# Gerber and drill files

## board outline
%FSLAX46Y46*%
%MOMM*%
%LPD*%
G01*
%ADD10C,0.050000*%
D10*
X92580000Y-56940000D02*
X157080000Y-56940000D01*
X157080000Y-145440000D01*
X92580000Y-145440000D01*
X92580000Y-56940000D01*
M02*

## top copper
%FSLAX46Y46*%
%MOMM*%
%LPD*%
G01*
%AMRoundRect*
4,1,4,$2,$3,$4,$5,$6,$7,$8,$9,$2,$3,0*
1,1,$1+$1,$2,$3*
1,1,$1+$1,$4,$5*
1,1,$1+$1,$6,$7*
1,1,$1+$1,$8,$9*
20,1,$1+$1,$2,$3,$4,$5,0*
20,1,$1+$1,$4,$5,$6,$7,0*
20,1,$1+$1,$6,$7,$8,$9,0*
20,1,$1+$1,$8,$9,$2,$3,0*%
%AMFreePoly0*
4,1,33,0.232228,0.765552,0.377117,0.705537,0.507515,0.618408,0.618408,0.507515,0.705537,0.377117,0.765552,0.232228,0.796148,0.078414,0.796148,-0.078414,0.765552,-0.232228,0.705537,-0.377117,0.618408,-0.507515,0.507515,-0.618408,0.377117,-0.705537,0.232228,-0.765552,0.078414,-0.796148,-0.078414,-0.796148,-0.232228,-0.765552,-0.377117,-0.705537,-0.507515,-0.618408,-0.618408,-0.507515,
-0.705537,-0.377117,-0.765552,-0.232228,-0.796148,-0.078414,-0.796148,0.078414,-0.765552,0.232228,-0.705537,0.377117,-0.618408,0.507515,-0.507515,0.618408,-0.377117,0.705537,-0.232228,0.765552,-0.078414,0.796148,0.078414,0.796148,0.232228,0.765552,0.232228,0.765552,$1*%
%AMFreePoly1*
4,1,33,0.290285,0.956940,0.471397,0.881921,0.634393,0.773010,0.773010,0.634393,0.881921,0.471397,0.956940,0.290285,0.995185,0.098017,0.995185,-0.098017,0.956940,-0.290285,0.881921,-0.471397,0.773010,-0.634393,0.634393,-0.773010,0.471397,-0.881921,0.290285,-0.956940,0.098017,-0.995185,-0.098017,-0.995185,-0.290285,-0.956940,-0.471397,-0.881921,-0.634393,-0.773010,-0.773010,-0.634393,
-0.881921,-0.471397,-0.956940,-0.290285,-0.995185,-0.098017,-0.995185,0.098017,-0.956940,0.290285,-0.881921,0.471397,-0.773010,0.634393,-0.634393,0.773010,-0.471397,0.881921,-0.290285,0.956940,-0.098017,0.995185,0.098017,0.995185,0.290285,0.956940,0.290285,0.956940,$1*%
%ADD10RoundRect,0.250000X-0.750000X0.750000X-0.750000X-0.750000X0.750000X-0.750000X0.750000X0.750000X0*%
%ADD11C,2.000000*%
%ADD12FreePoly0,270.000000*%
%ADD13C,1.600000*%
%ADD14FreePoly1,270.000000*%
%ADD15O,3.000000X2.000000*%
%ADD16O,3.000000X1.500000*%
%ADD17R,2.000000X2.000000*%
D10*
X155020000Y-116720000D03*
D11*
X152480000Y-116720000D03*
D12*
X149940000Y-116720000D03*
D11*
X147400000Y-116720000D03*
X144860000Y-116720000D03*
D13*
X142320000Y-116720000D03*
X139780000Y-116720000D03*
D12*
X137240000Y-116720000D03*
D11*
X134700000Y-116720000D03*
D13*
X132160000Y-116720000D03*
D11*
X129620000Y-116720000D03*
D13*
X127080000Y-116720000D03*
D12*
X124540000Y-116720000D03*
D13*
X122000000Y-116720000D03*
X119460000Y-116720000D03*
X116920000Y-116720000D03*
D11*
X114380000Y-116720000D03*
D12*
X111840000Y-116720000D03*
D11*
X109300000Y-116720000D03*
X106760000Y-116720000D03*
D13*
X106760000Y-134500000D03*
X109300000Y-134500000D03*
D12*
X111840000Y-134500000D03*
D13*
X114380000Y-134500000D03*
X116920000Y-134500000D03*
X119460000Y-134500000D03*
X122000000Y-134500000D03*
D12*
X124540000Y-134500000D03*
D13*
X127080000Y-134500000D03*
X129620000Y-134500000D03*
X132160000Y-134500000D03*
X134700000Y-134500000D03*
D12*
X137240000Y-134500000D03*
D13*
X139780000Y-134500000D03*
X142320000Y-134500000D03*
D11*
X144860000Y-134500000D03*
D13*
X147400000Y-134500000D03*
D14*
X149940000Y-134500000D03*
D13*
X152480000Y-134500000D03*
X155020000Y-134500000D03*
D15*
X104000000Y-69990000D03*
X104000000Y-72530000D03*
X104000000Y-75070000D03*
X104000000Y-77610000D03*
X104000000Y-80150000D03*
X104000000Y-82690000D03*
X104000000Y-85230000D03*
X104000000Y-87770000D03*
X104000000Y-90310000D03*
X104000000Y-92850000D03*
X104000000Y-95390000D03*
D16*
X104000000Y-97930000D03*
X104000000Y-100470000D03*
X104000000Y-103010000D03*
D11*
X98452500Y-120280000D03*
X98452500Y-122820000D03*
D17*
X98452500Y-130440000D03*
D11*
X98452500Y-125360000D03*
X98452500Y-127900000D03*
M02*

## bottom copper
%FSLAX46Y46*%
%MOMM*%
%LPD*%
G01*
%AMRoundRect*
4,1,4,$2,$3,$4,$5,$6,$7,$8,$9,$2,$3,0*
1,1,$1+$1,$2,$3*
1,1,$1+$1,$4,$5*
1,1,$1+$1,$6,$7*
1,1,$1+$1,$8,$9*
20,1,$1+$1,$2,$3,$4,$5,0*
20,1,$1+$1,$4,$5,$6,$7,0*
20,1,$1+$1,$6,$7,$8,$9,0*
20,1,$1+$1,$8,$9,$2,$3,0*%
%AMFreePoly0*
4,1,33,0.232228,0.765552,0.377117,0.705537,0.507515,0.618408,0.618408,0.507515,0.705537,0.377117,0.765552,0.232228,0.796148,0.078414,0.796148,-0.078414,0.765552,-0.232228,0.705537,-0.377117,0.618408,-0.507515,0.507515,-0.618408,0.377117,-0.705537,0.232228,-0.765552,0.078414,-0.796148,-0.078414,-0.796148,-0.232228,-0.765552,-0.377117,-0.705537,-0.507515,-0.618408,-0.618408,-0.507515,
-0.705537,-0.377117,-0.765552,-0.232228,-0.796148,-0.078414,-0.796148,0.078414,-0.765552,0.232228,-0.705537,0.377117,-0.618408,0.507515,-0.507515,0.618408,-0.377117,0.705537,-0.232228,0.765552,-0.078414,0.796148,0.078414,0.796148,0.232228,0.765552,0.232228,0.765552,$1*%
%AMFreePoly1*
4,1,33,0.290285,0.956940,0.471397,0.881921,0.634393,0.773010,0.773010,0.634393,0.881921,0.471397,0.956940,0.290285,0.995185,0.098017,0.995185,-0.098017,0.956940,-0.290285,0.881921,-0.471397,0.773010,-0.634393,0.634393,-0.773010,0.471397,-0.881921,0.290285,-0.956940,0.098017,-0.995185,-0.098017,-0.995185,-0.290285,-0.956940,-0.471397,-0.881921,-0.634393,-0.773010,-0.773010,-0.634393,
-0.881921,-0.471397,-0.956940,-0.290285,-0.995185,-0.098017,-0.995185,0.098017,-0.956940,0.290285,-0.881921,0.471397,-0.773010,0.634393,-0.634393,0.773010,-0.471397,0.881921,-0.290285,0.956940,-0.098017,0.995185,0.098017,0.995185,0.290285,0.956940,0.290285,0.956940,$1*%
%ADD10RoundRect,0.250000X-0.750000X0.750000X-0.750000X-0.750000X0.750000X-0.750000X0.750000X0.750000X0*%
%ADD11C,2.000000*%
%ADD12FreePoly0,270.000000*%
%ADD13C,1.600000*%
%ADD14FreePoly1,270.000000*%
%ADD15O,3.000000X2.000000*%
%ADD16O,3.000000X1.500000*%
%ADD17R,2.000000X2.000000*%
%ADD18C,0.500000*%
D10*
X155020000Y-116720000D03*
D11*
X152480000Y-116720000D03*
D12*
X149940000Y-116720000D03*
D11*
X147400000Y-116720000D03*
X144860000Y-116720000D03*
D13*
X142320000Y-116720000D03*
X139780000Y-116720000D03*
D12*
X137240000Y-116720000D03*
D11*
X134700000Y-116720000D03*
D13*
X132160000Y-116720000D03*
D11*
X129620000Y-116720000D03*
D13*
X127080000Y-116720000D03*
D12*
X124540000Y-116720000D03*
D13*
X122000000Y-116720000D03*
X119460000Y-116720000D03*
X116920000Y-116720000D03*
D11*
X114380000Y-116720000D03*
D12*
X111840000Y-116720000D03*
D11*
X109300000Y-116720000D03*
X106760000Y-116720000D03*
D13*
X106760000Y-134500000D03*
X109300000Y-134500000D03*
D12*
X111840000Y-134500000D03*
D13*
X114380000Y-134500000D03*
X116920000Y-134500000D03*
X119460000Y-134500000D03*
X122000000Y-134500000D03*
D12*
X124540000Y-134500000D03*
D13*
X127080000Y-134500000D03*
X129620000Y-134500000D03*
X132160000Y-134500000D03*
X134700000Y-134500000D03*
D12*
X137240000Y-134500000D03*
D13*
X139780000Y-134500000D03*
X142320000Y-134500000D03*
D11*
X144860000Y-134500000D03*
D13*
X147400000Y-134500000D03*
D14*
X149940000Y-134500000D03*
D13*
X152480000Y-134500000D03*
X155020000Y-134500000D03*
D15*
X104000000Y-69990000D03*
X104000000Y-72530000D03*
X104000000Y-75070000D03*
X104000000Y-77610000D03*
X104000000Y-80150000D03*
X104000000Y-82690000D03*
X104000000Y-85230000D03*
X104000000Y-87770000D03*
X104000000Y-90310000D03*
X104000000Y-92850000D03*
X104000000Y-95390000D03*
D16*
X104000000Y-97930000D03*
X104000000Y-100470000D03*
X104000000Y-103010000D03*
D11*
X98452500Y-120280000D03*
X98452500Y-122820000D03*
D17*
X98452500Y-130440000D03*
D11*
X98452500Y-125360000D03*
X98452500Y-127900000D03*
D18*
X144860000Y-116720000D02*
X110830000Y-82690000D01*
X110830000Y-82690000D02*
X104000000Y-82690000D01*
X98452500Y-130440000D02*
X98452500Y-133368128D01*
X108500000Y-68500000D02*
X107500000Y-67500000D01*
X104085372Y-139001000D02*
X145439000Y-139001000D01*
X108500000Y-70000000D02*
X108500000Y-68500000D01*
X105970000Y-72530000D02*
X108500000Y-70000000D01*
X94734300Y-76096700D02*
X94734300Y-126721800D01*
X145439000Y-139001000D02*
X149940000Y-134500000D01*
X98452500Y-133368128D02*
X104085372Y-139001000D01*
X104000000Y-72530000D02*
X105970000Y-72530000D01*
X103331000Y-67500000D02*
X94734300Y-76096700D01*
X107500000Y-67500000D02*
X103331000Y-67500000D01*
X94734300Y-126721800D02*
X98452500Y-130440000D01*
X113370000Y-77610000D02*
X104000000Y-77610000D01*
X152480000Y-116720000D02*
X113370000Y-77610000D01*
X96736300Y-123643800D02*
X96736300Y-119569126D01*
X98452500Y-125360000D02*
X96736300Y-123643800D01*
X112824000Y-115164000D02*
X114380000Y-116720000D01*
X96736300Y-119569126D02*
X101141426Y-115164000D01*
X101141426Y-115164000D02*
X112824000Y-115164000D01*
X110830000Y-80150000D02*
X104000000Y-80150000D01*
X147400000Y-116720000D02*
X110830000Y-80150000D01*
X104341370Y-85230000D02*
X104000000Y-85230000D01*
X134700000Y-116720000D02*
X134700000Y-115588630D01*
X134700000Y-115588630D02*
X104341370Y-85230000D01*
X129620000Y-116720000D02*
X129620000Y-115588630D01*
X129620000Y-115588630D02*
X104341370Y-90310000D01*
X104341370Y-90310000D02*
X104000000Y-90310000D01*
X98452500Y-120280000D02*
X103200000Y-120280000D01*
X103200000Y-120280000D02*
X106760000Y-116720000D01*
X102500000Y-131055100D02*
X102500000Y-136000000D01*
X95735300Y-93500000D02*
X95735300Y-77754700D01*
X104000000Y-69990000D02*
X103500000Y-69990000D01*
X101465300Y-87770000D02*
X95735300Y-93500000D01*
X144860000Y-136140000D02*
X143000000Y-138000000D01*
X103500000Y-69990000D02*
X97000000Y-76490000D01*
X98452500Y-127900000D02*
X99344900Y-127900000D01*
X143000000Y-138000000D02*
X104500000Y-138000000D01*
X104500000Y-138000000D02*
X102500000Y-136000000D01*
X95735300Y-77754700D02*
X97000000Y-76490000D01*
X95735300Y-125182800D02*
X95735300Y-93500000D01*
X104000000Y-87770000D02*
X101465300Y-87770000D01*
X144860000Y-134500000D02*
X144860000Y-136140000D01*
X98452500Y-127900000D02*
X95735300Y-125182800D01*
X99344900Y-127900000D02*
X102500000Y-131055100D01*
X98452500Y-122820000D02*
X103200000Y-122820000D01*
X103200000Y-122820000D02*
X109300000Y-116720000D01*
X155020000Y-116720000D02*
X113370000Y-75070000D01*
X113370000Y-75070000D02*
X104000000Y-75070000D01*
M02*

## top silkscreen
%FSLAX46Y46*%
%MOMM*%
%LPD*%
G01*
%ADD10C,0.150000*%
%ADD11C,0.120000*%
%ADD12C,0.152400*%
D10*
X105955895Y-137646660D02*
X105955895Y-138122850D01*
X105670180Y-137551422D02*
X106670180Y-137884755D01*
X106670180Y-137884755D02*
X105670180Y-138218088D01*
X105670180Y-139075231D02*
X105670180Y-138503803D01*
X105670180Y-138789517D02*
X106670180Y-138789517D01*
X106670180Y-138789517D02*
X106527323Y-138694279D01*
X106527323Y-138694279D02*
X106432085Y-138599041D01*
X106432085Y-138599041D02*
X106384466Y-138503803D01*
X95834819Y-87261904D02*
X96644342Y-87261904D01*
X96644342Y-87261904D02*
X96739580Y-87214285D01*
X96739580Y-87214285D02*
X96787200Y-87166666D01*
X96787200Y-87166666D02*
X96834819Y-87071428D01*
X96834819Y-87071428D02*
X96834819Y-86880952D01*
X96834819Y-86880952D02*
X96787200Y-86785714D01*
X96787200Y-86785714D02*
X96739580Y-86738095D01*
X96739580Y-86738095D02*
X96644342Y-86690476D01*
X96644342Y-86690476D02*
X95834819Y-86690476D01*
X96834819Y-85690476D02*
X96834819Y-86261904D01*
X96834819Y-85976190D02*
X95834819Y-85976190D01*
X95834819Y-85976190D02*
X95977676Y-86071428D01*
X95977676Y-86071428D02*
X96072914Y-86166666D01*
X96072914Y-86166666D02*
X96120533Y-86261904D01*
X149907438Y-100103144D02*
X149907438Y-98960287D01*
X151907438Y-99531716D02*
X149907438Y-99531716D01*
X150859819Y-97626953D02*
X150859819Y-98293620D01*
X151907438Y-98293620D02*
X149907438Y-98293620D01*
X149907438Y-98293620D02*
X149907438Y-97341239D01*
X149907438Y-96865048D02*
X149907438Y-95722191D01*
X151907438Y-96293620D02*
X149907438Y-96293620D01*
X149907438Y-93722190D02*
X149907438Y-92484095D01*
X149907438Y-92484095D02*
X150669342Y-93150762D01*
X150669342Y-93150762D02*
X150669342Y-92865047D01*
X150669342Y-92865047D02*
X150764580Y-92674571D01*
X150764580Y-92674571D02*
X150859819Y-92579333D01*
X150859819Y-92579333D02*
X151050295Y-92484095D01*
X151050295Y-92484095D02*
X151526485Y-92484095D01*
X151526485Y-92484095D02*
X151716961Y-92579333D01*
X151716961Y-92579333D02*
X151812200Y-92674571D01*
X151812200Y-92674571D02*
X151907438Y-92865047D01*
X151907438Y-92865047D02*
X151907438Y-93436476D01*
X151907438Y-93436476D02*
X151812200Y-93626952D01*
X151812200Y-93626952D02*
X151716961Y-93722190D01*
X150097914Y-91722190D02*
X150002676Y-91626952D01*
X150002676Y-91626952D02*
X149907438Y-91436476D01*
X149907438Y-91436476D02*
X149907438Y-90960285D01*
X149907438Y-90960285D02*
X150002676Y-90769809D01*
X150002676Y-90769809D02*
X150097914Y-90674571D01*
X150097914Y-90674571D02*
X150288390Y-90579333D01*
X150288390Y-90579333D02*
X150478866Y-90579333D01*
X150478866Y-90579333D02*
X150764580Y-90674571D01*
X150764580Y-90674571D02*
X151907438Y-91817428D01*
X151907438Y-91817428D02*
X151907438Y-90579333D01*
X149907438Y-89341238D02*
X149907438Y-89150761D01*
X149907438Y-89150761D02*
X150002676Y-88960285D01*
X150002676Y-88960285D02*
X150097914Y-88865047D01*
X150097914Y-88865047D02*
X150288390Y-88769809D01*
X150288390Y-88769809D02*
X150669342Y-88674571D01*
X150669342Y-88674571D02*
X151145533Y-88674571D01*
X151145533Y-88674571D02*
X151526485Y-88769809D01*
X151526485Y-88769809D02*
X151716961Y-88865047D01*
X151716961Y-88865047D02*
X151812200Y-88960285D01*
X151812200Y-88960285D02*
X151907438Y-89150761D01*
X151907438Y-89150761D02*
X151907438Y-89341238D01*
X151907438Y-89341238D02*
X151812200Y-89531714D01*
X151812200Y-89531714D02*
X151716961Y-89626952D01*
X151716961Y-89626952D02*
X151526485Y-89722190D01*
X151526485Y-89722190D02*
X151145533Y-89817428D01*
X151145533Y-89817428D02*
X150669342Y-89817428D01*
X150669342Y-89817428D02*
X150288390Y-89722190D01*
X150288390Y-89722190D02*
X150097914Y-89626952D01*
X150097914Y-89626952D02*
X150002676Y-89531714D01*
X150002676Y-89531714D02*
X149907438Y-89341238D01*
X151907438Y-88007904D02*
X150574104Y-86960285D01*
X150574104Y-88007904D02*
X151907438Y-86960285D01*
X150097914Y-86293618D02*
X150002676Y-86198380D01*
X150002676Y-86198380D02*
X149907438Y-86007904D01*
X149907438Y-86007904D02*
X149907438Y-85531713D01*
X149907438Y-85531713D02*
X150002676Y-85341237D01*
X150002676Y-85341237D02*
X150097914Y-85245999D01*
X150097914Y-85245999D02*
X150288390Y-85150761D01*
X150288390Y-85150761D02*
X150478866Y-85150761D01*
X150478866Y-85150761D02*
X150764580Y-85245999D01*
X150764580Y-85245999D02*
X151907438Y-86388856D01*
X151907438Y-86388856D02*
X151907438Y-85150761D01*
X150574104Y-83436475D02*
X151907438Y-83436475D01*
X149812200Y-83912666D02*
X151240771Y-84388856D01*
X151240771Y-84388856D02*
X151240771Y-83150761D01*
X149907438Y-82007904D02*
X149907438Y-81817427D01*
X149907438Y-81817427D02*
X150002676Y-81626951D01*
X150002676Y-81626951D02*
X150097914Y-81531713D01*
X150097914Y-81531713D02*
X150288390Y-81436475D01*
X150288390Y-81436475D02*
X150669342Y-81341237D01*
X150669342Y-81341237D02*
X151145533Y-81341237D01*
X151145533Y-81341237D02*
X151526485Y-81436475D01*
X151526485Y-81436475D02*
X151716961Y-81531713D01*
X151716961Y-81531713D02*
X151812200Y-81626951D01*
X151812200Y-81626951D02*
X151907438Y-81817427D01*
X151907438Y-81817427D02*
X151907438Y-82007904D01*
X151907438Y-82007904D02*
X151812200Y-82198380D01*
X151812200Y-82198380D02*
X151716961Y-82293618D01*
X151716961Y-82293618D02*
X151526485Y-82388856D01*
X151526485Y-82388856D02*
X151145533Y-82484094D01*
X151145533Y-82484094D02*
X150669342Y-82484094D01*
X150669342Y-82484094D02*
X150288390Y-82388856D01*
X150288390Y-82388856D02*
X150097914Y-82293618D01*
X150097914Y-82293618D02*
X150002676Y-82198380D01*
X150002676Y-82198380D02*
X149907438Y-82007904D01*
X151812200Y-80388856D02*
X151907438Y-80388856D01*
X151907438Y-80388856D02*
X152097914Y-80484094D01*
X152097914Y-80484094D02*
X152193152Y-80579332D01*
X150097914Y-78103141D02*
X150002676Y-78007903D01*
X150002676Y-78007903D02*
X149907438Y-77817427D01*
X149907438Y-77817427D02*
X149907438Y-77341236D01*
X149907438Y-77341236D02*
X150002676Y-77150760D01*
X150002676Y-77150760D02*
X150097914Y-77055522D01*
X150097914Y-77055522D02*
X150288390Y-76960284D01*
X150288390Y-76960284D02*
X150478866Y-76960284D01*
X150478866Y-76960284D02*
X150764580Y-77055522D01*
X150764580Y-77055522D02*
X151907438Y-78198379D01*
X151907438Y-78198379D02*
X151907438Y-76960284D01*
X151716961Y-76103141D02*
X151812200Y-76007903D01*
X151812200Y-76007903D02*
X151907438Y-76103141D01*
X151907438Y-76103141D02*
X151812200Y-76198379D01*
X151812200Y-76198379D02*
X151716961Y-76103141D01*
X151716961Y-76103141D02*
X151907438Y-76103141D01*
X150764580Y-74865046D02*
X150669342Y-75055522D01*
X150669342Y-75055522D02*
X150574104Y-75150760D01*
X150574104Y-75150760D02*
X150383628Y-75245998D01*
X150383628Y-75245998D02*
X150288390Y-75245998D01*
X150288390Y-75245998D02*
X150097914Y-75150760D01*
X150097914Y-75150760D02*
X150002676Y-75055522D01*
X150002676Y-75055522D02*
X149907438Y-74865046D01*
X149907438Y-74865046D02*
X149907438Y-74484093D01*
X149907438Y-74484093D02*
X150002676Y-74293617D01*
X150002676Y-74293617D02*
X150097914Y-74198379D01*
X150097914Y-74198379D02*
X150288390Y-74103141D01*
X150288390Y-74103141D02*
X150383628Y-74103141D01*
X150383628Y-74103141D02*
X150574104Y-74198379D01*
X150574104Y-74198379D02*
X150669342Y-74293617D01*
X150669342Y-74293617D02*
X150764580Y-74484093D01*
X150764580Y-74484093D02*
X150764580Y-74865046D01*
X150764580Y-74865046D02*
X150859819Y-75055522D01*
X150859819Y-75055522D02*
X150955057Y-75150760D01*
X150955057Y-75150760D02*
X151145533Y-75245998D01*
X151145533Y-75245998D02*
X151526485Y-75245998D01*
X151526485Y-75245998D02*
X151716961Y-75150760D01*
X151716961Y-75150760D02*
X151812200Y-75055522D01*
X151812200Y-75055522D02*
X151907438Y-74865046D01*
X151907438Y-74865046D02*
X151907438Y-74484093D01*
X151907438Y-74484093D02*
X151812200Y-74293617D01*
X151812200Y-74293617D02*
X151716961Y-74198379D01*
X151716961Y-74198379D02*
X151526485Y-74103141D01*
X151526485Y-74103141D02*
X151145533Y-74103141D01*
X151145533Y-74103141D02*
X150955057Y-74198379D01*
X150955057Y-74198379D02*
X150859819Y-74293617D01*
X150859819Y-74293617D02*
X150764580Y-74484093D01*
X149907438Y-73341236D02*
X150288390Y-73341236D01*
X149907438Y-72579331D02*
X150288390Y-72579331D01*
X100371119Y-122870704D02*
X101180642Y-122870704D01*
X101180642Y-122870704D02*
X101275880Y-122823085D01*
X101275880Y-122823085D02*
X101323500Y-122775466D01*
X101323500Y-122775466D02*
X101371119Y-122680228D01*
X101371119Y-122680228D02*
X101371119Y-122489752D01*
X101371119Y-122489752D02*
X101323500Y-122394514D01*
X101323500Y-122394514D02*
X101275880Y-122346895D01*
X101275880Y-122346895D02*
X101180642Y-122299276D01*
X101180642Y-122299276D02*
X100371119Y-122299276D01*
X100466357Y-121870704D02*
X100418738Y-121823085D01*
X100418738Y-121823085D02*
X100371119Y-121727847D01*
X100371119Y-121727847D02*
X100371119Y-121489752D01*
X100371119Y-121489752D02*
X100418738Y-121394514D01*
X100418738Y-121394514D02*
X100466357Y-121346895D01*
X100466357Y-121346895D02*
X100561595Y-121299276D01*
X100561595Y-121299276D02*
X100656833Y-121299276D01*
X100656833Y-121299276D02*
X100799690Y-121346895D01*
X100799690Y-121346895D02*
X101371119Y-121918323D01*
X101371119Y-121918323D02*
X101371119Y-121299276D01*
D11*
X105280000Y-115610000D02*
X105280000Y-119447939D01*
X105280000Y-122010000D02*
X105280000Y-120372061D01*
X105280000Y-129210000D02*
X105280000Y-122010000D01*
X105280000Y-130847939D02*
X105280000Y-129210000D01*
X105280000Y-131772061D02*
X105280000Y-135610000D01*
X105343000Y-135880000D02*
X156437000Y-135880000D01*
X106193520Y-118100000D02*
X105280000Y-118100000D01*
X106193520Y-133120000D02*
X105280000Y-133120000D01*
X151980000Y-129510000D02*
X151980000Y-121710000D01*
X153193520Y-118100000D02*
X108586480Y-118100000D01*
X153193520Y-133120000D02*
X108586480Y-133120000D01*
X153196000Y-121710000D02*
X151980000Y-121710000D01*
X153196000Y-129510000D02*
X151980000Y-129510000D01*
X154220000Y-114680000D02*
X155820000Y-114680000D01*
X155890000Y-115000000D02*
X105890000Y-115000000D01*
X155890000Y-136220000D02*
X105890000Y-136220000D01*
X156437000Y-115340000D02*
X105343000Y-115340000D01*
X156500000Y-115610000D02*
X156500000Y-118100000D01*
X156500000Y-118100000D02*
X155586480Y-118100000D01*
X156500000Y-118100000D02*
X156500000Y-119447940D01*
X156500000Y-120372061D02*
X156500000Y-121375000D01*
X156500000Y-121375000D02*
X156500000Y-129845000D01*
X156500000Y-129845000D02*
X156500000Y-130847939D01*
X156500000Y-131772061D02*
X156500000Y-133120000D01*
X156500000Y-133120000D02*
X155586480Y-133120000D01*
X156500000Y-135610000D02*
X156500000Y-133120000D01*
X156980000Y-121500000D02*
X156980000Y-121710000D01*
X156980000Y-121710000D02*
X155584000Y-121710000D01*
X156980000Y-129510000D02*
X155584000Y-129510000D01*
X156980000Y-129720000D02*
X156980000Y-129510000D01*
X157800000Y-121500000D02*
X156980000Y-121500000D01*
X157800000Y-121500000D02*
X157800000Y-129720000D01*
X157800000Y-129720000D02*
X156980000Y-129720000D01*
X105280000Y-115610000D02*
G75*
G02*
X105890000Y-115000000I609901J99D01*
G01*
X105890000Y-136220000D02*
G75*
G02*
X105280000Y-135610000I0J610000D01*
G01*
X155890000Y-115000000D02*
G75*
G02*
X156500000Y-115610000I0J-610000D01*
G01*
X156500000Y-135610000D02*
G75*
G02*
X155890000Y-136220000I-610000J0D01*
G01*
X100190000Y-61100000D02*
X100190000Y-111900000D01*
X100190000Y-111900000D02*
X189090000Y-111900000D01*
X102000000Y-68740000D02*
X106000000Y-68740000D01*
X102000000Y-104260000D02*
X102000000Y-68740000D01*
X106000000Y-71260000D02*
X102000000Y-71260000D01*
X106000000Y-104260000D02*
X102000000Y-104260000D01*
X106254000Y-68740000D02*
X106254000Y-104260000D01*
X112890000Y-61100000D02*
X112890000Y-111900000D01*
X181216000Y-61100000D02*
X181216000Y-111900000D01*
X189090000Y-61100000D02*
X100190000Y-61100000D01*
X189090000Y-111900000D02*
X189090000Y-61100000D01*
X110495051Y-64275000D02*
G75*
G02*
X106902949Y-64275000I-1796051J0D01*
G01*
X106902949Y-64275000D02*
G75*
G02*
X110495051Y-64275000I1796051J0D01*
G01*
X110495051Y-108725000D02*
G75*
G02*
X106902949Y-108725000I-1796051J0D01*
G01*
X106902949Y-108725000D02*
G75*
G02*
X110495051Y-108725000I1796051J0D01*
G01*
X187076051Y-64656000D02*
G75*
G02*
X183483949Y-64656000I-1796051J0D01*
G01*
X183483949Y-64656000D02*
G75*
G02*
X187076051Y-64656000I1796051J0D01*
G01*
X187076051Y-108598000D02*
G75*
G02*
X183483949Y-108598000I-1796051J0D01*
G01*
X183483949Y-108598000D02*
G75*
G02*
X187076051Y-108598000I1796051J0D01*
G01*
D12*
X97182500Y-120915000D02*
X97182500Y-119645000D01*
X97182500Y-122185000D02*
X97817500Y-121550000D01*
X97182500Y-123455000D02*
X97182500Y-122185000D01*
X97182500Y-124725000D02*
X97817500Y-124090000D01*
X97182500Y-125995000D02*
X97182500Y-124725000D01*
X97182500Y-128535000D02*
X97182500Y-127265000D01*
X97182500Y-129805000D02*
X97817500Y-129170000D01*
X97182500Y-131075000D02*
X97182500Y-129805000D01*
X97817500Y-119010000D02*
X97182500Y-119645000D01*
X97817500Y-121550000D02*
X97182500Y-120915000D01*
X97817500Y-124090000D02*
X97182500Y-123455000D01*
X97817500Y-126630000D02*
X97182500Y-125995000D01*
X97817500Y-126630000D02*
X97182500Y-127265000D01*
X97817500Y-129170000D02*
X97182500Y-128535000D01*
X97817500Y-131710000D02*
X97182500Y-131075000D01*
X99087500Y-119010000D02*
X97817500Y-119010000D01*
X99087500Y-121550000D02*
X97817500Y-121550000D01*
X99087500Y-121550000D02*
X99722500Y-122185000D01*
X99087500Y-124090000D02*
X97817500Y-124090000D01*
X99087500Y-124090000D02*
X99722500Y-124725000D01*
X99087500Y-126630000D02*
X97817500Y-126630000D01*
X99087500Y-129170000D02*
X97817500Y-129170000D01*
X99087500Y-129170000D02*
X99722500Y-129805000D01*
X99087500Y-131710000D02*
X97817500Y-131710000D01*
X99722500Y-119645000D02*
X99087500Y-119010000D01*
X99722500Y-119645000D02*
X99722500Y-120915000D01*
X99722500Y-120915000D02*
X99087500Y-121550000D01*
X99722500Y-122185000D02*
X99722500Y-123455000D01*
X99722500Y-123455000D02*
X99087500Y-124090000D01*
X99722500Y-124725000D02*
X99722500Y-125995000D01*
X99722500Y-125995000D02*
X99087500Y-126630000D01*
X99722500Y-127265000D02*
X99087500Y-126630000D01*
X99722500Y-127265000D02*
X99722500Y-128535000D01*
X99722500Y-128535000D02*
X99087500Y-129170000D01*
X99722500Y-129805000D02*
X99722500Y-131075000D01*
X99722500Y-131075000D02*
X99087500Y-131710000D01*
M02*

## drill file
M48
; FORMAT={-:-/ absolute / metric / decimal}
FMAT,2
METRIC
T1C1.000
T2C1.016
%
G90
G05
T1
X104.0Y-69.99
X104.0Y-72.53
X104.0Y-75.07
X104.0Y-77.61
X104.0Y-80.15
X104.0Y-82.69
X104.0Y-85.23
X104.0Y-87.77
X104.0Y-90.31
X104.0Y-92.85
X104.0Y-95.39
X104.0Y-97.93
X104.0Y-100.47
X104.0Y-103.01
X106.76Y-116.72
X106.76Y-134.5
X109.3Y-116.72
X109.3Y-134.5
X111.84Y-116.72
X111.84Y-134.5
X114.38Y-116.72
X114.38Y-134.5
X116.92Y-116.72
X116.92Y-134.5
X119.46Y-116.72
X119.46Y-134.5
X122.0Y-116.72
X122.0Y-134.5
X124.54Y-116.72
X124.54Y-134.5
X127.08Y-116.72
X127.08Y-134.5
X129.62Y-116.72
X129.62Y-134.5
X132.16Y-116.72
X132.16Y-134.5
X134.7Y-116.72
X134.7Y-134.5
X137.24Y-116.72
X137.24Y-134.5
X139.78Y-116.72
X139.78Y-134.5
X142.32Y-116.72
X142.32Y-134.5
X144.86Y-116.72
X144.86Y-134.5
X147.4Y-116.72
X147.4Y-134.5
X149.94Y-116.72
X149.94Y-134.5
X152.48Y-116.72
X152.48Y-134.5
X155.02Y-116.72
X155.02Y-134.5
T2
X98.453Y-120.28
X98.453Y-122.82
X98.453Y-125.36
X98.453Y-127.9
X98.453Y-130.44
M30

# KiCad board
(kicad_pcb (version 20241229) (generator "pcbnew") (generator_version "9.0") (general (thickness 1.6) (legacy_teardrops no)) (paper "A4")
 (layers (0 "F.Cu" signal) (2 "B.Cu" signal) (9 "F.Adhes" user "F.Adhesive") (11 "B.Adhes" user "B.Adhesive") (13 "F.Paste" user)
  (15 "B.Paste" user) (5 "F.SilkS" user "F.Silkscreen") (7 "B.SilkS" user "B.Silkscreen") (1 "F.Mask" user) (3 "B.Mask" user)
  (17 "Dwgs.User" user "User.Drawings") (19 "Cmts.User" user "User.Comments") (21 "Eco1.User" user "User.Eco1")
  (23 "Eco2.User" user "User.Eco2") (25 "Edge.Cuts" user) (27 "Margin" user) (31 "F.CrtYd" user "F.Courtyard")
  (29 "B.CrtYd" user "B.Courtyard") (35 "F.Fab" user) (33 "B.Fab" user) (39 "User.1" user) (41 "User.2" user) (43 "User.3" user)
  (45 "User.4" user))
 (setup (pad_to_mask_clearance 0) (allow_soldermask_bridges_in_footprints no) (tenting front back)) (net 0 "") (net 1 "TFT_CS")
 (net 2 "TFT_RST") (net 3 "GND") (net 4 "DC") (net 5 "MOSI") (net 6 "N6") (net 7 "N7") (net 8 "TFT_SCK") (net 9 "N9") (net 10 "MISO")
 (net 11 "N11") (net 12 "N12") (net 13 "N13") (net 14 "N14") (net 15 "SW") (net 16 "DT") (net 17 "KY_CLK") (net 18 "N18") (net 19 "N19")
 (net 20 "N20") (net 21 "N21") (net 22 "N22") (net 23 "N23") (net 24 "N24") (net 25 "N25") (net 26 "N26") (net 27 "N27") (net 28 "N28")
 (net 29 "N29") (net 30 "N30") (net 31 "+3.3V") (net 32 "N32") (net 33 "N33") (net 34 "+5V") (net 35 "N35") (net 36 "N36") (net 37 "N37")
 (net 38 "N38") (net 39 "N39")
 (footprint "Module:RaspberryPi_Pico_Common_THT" (layer "F.Cu") (at 155.02 116.72 -90)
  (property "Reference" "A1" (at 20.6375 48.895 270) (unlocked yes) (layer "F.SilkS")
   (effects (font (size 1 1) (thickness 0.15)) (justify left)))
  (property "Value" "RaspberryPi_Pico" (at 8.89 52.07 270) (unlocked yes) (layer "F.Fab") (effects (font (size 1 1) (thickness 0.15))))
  (fp_line (start -1.11 49.74) (end 2.727939 49.74) (stroke (width 0.12) (type solid)) (layer "F.SilkS"))
  (fp_line (start 5.29 49.74) (end 3.652061 49.74) (stroke (width 0.12) (type solid)) (layer "F.SilkS"))
  (fp_line (start 12.49 49.74) (end 5.29 49.74) (stroke (width 0.12) (type solid)) (layer "F.SilkS"))
  (fp_line (start 14.127939 49.74) (end 12.49 49.74) (stroke (width 0.12) (type solid)) (layer "F.SilkS"))
  (fp_line (start 15.052061 49.74) (end 18.89 49.74) (stroke (width 0.12) (type solid)) (layer "F.SilkS"))
  (fp_line (start 19.16 49.677) (end 19.16 -1.417) (stroke (width 0.12) (type solid)) (layer "F.SilkS"))
  (fp_line (start 1.38 48.82648) (end 1.38 49.74) (stroke (width 0.12) (type solid)) (layer "F.SilkS"))
  (fp_line (start 16.4 48.82648) (end 16.4 49.74) (stroke (width 0.12) (type solid)) (layer "F.SilkS"))
  (fp_line (start 12.79 3.04) (end 4.99 3.04) (stroke (width 0.12) (type solid)) (layer "F.SilkS"))
  (fp_line (start 1.38 1.82648) (end 1.38 46.43352) (stroke (width 0.12) (type solid)) (layer "F.SilkS"))
  (fp_line (start 16.4 1.82648) (end 16.4 46.43352) (stroke (width 0.12) (type solid)) (layer "F.SilkS"))
  (fp_line (start 4.99 1.824) (end 4.99 3.04) (stroke (width 0.12) (type solid)) (layer "F.SilkS"))
  (fp_line (start 12.79 1.824) (end 12.79 3.04) (stroke (width 0.12) (type solid)) (layer "F.SilkS"))
  (fp_line (start -2.04 0.8) (end -2.04 -0.8) (stroke (width 0.12) (type solid)) (layer "F.SilkS"))
  (fp_line (start -1.72 -0.87) (end -1.72 49.13) (stroke (width 0.12) (type solid)) (layer "F.SilkS"))
  (fp_line (start 19.5 -0.87) (end 19.5 49.13) (stroke (width 0.12) (type solid)) (layer "F.SilkS"))
  (fp_line (start -1.38 -1.417) (end -1.38 49.677) (stroke (width 0.12) (type solid)) (layer "F.SilkS"))
  (fp_line (start -1.11 -1.48) (end 1.38 -1.48) (stroke (width 0.12) (type solid)) (layer "F.SilkS"))
  (fp_line (start 1.38 -1.48) (end 1.38 -0.56648) (stroke (width 0.12) (type solid)) (layer "F.SilkS"))
  (fp_line (start 1.38 -1.48) (end 2.72794 -1.48) (stroke (width 0.12) (type solid)) (layer "F.SilkS"))
  (fp_line (start 3.652061 -1.48) (end 4.655 -1.48) (stroke (width 0.12) (type solid)) (layer "F.SilkS"))
  (fp_line (start 4.655 -1.48) (end 13.125 -1.48) (stroke (width 0.12) (type solid)) (layer "F.SilkS"))
  (fp_line (start 13.125 -1.48) (end 14.127939 -1.48) (stroke (width 0.12) (type solid)) (layer "F.SilkS"))
  (fp_line (start 15.052061 -1.48) (end 16.4 -1.48) (stroke (width 0.12) (type solid)) (layer "F.SilkS"))
  (fp_line (start 16.4 -1.48) (end 16.4 -0.56648) (stroke (width 0.12) (type solid)) (layer "F.SilkS"))
  (fp_line (start 18.89 -1.48) (end 16.4 -1.48) (stroke (width 0.12) (type solid)) (layer "F.SilkS"))
  (fp_line (start 4.78 -1.96) (end 4.99 -1.96) (stroke (width 0.12) (type solid)) (layer "F.SilkS"))
  (fp_line (start 4.99 -1.96) (end 4.99 -0.564) (stroke (width 0.12) (type solid)) (layer "F.SilkS"))
  (fp_line (start 12.79 -1.96) (end 12.79 -0.564) (stroke (width 0.12) (type solid)) (layer "F.SilkS"))
  (fp_line (start 13 -1.96) (end 12.79 -1.96) (stroke (width 0.12) (type solid)) (layer "F.SilkS"))
  (fp_line (start 4.78 -2.78) (end 4.78 -1.96) (stroke (width 0.12) (type solid)) (layer "F.SilkS"))
  (fp_line (start 4.78 -2.78) (end 13 -2.78) (stroke (width 0.12) (type solid)) (layer "F.SilkS"))
  (fp_line (start 13 -2.78) (end 13 -1.96) (stroke (width 0.12) (type solid)) (layer "F.SilkS"))
  (fp_arc (start -1.11 49.74) (mid -1.541364 49.561364) (end -1.72 49.13) (stroke (width 0.12) (type solid)) (layer "F.SilkS"))
  (fp_arc (start 19.5 49.13) (mid 19.321335 49.561335) (end 18.89 49.74) (stroke (width 0.12) (type solid)) (layer "F.SilkS"))
  (fp_arc (start -1.72 -0.87) (mid -1.541335 -1.301335) (end -1.11 -1.48) (stroke (width 0.12) (type solid)) (layer "F.SilkS"))
  (fp_arc (start 18.89 -1.48) (mid 19.321335 -1.301335) (end 19.5 -0.87) (stroke (width 0.12) (type solid)) (layer "F.SilkS"))
  (pad "1" thru_hole roundrect (at 0 0 270) (size 2 2) (drill 1) (layers "*.Cu" "*.Mask") (remove_unused_layers no) (roundrect_rratio 0.125)
   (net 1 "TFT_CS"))
  (pad "2" thru_hole circle (at 0 2.54 270) (size 2 2) (drill 1) (layers "*.Cu" "*.Mask") (remove_unused_layers no) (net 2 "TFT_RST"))
  (pad "3" thru_hole custom (at 0 5.08 270) (size 1.6 1.6) (drill 1) (layers "*.Cu" "*.Mask") (remove_unused_layers no) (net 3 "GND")
   (options (clearance outline) (anchor circle)) (primitives))
  (pad "4" thru_hole circle (at 0 7.62 270) (size 2 2) (drill 1) (layers "*.Cu" "*.Mask") (remove_unused_layers no) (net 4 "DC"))
  (pad "5" thru_hole circle (at 0 10.16 270) (size 2 2) (drill 1) (layers "*.Cu" "*.Mask") (remove_unused_layers no) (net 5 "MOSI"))
  (pad "6" thru_hole circle (at 0 12.7 270) (size 1.6 1.6) (drill 1) (layers "*.Cu" "*.Mask") (remove_unused_layers no) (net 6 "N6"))
  (pad "7" thru_hole circle (at 0 15.24 270) (size 1.6 1.6) (drill 1) (layers "*.Cu" "*.Mask") (remove_unused_layers no) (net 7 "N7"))
  (pad "8" thru_hole custom (at 0 17.78 270) (size 1.6 1.6) (drill 1) (layers "*.Cu" "*.Mask") (remove_unused_layers no) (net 3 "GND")
   (options (clearance outline) (anchor circle)) (primitives))
  (pad "9" thru_hole circle (at 0 20.32 270) (size 2 2) (drill 1) (layers "*.Cu" "*.Mask") (remove_unused_layers no) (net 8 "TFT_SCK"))
  (pad "10" thru_hole circle (at 0 22.86 270) (size 1.6 1.6) (drill 1) (layers "*.Cu" "*.Mask") (remove_unused_layers no) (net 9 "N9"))
  (pad "11" thru_hole circle (at 0 25.4 270) (size 2 2) (drill 1) (layers "*.Cu" "*.Mask") (remove_unused_layers no) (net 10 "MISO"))
  (pad "12" thru_hole circle (at 0 27.94 270) (size 1.6 1.6) (drill 1) (layers "*.Cu" "*.Mask") (remove_unused_layers no) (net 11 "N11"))
  (pad "13" thru_hole custom (at 0 30.48 270) (size 1.6 1.6) (drill 1) (layers "*.Cu" "*.Mask") (remove_unused_layers no) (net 3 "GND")
   (options (clearance outline) (anchor circle)) (primitives))
  (pad "14" thru_hole circle (at 0 33.02 270) (size 1.6 1.6) (drill 1) (layers "*.Cu" "*.Mask") (remove_unused_layers no) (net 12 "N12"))
  (pad "15" thru_hole circle (at 0 35.56 270) (size 1.6 1.6) (drill 1) (layers "*.Cu" "*.Mask") (remove_unused_layers no) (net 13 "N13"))
  (pad "16" thru_hole circle (at 0 38.1 270) (size 1.6 1.6) (drill 1) (layers "*.Cu" "*.Mask") (remove_unused_layers no) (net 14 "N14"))
  (pad "17" thru_hole circle (at 0 40.64 270) (size 2 2) (drill 1) (layers "*.Cu" "*.Mask") (remove_unused_layers no) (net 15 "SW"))
  (pad "18" thru_hole custom (at 0 43.18 270) (size 1.6 1.6) (drill 1) (layers "*.Cu" "*.Mask") (remove_unused_layers no) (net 3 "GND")
   (options (clearance outline) (anchor circle)) (primitives))
  (pad "19" thru_hole circle (at 0 45.72 270) (size 2 2) (drill 1) (layers "*.Cu" "*.Mask") (remove_unused_layers no) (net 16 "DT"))
  (pad "20" thru_hole circle (at 0 48.26 270) (size 2 2) (drill 1) (layers "*.Cu" "*.Mask") (remove_unused_layers no) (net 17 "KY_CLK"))
  (pad "21" thru_hole circle (at 17.78 48.26 270) (size 1.6 1.6) (drill 1) (layers "*.Cu" "*.Mask") (remove_unused_layers no) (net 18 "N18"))
  (pad "22" thru_hole circle (at 17.78 45.72 270) (size 1.6 1.6) (drill 1) (layers "*.Cu" "*.Mask") (remove_unused_layers no) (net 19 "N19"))
  (pad "23" thru_hole custom (at 17.78 43.18 270) (size 1.6 1.6) (drill 1) (layers "*.Cu" "*.Mask") (remove_unused_layers no) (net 3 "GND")
   (options (clearance outline) (anchor circle)) (primitives))
  (pad "24" thru_hole circle (at 17.78 40.64 270) (size 1.6 1.6) (drill 1) (layers "*.Cu" "*.Mask") (remove_unused_layers no) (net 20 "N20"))
  (pad "25" thru_hole circle (at 17.78 38.1 270) (size 1.6 1.6) (drill 1) (layers "*.Cu" "*.Mask") (remove_unused_layers no) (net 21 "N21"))
  (pad "26" thru_hole circle (at 17.78 35.56 270) (size 1.6 1.6) (drill 1) (layers "*.Cu" "*.Mask") (remove_unused_layers no) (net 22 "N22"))
  (pad "27" thru_hole circle (at 17.78 33.02 270) (size 1.6 1.6) (drill 1) (layers "*.Cu" "*.Mask") (remove_unused_layers no) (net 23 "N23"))
  (pad "28" thru_hole custom (at 17.78 30.48 270) (size 1.6 1.6) (drill 1) (layers "*.Cu" "*.Mask") (remove_unused_layers no) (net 3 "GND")
   (options (clearance outline) (anchor circle)) (primitives))
  (pad "29" thru_hole circle (at 17.78 27.94 270) (size 1.6 1.6) (drill 1) (layers "*.Cu" "*.Mask") (remove_unused_layers no) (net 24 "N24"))
  (pad "30" thru_hole circle (at 17.78 25.4 270) (size 1.6 1.6) (drill 1) (layers "*.Cu" "*.Mask") (remove_unused_layers no) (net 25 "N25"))
  (pad "31" thru_hole circle (at 17.78 22.86 270) (size 1.6 1.6) (drill 1) (layers "*.Cu" "*.Mask") (remove_unused_layers no) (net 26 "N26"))
  (pad "32" thru_hole circle (at 17.78 20.32 270) (size 1.6 1.6) (drill 1) (layers "*.Cu" "*.Mask") (remove_unused_layers no) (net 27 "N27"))
  (pad "33" thru_hole custom (at 17.78 17.78 270) (size 1.6 1.6) (drill 1) (layers "*.Cu" "*.Mask") (remove_unused_layers no) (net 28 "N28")
   (options (clearance outline) (anchor circle)) (primitives))
  (pad "34" thru_hole circle (at 17.78 15.24 270) (size 1.6 1.6) (drill 1) (layers "*.Cu" "*.Mask") (remove_unused_layers no) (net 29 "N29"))
  (pad "35" thru_hole circle (at 17.78 12.7 270) (size 1.6 1.6) (drill 1) (layers "*.Cu" "*.Mask") (remove_unused_layers no) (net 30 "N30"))
  (pad "36" thru_hole circle (at 17.78 10.16 270) (size 2 2) (drill 1) (layers "*.Cu" "*.Mask") (remove_unused_layers no) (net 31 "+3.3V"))
  (pad "37" thru_hole circle (at 17.78 7.62 270) (size 1.6 1.6) (drill 1) (layers "*.Cu" "*.Mask") (remove_unused_layers no) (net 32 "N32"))
  (pad "38" thru_hole custom (at 17.78 5.08 270) (size 2 2) (drill 1) (layers "*.Cu" "*.Mask") (remove_unused_layers no) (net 3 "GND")
   (options (clearance outline) (anchor circle)) (primitives))
  (pad "39" thru_hole circle (at 17.78 2.54 270) (size 1.6 1.6) (drill 1) (layers "*.Cu" "*.Mask") (remove_unused_layers no) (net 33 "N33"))
  (pad "40" thru_hole circle (at 17.78 0 270) (size 1.6 1.6) (drill 1) (layers "*.Cu" "*.Mask") (remove_unused_layers no) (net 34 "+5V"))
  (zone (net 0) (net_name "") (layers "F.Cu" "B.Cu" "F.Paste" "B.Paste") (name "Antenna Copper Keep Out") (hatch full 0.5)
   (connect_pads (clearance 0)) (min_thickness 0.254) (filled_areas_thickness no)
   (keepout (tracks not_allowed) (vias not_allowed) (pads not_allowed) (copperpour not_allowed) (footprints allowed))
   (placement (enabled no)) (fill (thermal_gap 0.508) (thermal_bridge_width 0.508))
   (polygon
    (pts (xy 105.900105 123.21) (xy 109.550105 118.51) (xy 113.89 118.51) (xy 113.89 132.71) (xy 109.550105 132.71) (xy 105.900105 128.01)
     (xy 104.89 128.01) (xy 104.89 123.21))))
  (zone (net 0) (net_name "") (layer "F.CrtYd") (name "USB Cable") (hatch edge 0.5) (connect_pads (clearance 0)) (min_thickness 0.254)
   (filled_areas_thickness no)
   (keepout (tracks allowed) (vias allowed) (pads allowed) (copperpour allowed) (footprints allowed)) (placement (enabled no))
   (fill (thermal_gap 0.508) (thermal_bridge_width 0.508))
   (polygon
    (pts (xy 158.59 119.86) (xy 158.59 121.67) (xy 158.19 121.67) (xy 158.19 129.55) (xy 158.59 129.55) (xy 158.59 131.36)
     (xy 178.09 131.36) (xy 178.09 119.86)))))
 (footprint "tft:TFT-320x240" (layer "F.Cu") (at 104 86.5 -90)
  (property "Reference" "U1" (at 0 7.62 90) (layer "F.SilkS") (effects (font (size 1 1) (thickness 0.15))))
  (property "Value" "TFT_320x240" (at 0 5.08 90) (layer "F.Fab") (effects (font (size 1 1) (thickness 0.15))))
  (fp_line (start -25.4 3.81) (end 25.4 3.81) (stroke (width 0.12) (type solid)) (layer "F.SilkS"))
  (fp_line (start 25.4 3.81) (end 25.4 -85.09) (stroke (width 0.12) (type solid)) (layer "F.SilkS"))
  (fp_line (start -17.76 2) (end -17.76 -2) (stroke (width 0.12) (type solid)) (layer "F.SilkS"))
  (fp_line (start 17.76 2) (end -17.76 2) (stroke (width 0.12) (type solid)) (layer "F.SilkS"))
  (fp_line (start -15.24 -2) (end -15.24 2) (stroke (width 0.12) (type solid)) (layer "F.SilkS"))
  (fp_line (start 17.76 -2) (end 17.76 2) (stroke (width 0.12) (type solid)) (layer "F.SilkS"))
  (fp_line (start -17.76 -2.254) (end 17.76 -2.254) (stroke (width 0.12) (type solid)) (layer "F.SilkS"))
  (fp_line (start -25.4 -8.89) (end 25.4 -8.89) (stroke (width 0.12) (type solid)) (layer "F.SilkS"))
  (fp_line (start -25.4 -77.216) (end 25.4 -77.216) (stroke (width 0.12) (type solid)) (layer "F.SilkS"))
  (fp_line (start -25.4 -85.09) (end -25.4 3.81) (stroke (width 0.12) (type solid)) (layer "F.SilkS"))
  (fp_line (start 25.4 -85.09) (end -25.4 -85.09) (stroke (width 0.12) (type solid)) (layer "F.SilkS"))
  (fp_circle (center -22.225 -4.699) (end -23.495 -3.429) (stroke (width 0.12) (type solid)) (fill no) (layer "F.SilkS"))
  (fp_circle (center 22.225 -4.699) (end 20.955 -3.429) (stroke (width 0.12) (type solid)) (fill no) (layer "F.SilkS"))
  (fp_circle (center -21.844 -81.28) (end -23.114 -82.55) (stroke (width 0.12) (type solid)) (fill no) (layer "F.SilkS"))
  (fp_circle (center 22.098 -81.28) (end 20.828 -80.01) (stroke (width 0.12) (type solid)) (fill no) (layer "F.SilkS"))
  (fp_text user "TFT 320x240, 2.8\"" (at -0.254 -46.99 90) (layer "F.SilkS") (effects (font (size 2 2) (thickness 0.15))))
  (pad "1" thru_hole oval (at -16.51 0 270) (size 2 3) (drill 1) (layers "*.Cu" "*.Mask") (remove_unused_layers no) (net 31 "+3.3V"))
  (pad "2" thru_hole oval (at -13.97 0 270) (size 2 3) (drill 1) (layers "*.Cu" "*.Mask") (remove_unused_layers no) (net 3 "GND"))
  (pad "3" thru_hole oval (at -11.43 0 270) (size 2 3) (drill 1) (layers "*.Cu" "*.Mask") (remove_unused_layers no) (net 1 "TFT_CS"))
  (pad "4" thru_hole oval (at -8.89 0 270) (size 2 3) (drill 1) (layers "*.Cu" "*.Mask") (remove_unused_layers no) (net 2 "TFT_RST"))
  (pad "5" thru_hole oval (at -6.35 0 270) (size 2 3) (drill 1) (layers "*.Cu" "*.Mask") (remove_unused_layers no) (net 4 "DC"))
  (pad "6" thru_hole oval (at -3.81 0 270) (size 2 3) (drill 1) (layers "*.Cu" "*.Mask") (remove_unused_layers no) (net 5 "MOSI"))
  (pad "7" thru_hole oval (at -1.27 0 270) (size 2 3) (drill 1) (layers "*.Cu" "*.Mask") (remove_unused_layers no) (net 8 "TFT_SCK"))
  (pad "8" thru_hole oval (at 1.27 0 270) (size 2 3) (drill 1) (layers "*.Cu" "*.Mask") (remove_unused_layers no) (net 31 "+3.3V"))
  (pad "9" thru_hole oval (at 3.81 0 270) (size 2 3) (drill 1) (layers "*.Cu" "*.Mask") (remove_unused_layers no) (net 10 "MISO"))
  (pad "10" thru_hole oval (at 6.35 0 270) (size 2 3) (drill 1) (layers "*.Cu" "*.Mask") (remove_unused_layers no) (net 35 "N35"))
  (pad "11" thru_hole oval (at 8.89 0 270) (size 2 3) (drill 1) (layers "*.Cu" "*.Mask") (remove_unused_layers no) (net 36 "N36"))
  (pad "12" thru_hole oval (at 11.43 0 270) (size 1.5 3) (drill 1) (layers "*.Cu" "*.Mask") (remove_unused_layers no) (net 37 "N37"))
  (pad "13" thru_hole oval (at 13.97 0 270) (size 1.5 3) (drill 1) (layers "*.Cu" "*.Mask") (remove_unused_layers no) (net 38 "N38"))
  (pad "14" thru_hole oval (at 16.51 0 270) (size 1.5 3) (drill 1) (layers "*.Cu" "*.Mask") (remove_unused_layers no) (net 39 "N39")))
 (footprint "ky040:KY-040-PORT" (layer "F.Cu") (at 98.4525 126.63 -90)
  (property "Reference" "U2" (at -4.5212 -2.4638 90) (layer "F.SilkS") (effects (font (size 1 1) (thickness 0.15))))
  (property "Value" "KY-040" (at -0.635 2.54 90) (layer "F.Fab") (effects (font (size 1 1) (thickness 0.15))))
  (fp_line (start -5.715 1.27) (end -6.985 1.27) (stroke (width 0.1524) (type solid)) (layer "F.SilkS"))
  (fp_line (start -4.445 1.27) (end -5.08 0.635) (stroke (width 0.1524) (type solid)) (layer "F.SilkS"))
  (fp_line (start -3.175 1.27) (end -4.445 1.27) (stroke (width 0.1524) (type solid)) (layer "F.SilkS"))
  (fp_line (start -1.905 1.27) (end -2.54 0.635) (stroke (width 0.1524) (type solid)) (layer "F.SilkS"))
  (fp_line (start -0.635 1.27) (end -1.905 1.27) (stroke (width 0.1524) (type solid)) (layer "F.SilkS"))
  (fp_line (start 1.905 1.27) (end 0.635 1.27) (stroke (width 0.1524) (type solid)) (layer "F.SilkS"))
  (fp_line (start 3.175 1.27) (end 2.54 0.635) (stroke (width 0.1524) (type solid)) (layer "F.SilkS"))
  (fp_line (start 4.445 1.27) (end 3.175 1.27) (stroke (width 0.1524) (type solid)) (layer "F.SilkS"))
  (fp_line (start -7.62 0.635) (end -6.985 1.27) (stroke (width 0.1524) (type solid)) (layer "F.SilkS"))
  (fp_line (start -5.08 0.635) (end -5.715 1.27) (stroke (width 0.1524) (type solid)) (layer "F.SilkS"))
  (fp_line (start -2.54 0.635) (end -3.175 1.27) (stroke (width 0.1524) (type solid)) (layer "F.SilkS"))
  (fp_line (start 0 0.635) (end -0.635 1.27) (stroke (width 0.1524) (type solid)) (layer "F.SilkS"))
  (fp_line (start 0 0.635) (end 0.635 1.27) (stroke (width 0.1524) (type solid)) (layer "F.SilkS"))
  (fp_line (start 2.54 0.635) (end 1.905 1.27) (stroke (width 0.1524) (type solid)) (layer "F.SilkS"))
  (fp_line (start 5.08 0.635) (end 4.445 1.27) (stroke (width 0.1524) (type solid)) (layer "F.SilkS"))
  (fp_line (start -7.62 -0.635) (end -7.62 0.635) (stroke (width 0.1524) (type solid)) (layer "F.SilkS"))
  (fp_line (start -5.08 -0.635) (end -5.08 0.635) (stroke (width 0.1524) (type solid)) (layer "F.SilkS"))
  (fp_line (start -5.08 -0.635) (end -4.445 -1.27) (stroke (width 0.1524) (type solid)) (layer "F.SilkS"))
  (fp_line (start -2.54 -0.635) (end -2.54 0.635) (stroke (width 0.1524) (type solid)) (layer "F.SilkS"))
  (fp_line (start -2.54 -0.635) (end -1.905 -1.27) (stroke (width 0.1524) (type solid)) (layer "F.SilkS"))
  (fp_line (start 0 -0.635) (end 0 0.635) (stroke (width 0.1524) (type solid)) (layer "F.SilkS"))
  (fp_line (start 2.54 -0.635) (end 2.54 0.635) (stroke (width 0.1524) (type solid)) (layer "F.SilkS"))
  (fp_line (start 2.54 -0.635) (end 3.175 -1.27) (stroke (width 0.1524) (type solid)) (layer "F.SilkS"))
  (fp_line (start 5.08 -0.635) (end 5.08 0.635) (stroke (width 0.1524) (type solid)) (layer "F.SilkS"))
  (fp_line (start -6.985 -1.27) (end -7.62 -0.635) (stroke (width 0.1524) (type solid)) (layer "F.SilkS"))
  (fp_line (start -6.985 -1.27) (end -5.715 -1.27) (stroke (width 0.1524) (type solid)) (layer "F.SilkS"))
  (fp_line (start -5.715 -1.27) (end -5.08 -0.635) (stroke (width 0.1524) (type solid)) (layer "F.SilkS"))
  (fp_line (start -4.445 -1.27) (end -3.175 -1.27) (stroke (width 0.1524) (type solid)) (layer "F.SilkS"))
  (fp_line (start -3.175 -1.27) (end -2.54 -0.635) (stroke (width 0.1524) (type solid)) (layer "F.SilkS"))
  (fp_line (start -1.905 -1.27) (end -0.635 -1.27) (stroke (width 0.1524) (type solid)) (layer "F.SilkS"))
  (fp_line (start -0.635 -1.27) (end 0 -0.635) (stroke (width 0.1524) (type solid)) (layer "F.SilkS"))
  (fp_line (start 0.635 -1.27) (end 0 -0.635) (stroke (width 0.1524) (type solid)) (layer "F.SilkS"))
  (fp_line (start 0.635 -1.27) (end 1.905 -1.27) (stroke (width 0.1524) (type solid)) (layer "F.SilkS"))
  (fp_line (start 1.905 -1.27) (end 2.54 -0.635) (stroke (width 0.1524) (type solid)) (layer "F.SilkS"))
  (fp_line (start 3.175 -1.27) (end 4.445 -1.27) (stroke (width 0.1524) (type solid)) (layer "F.SilkS"))
  (fp_line (start 4.445 -1.27) (end 5.08 -0.635) (stroke (width 0.1524) (type solid)) (layer "F.SilkS"))
  (pad "CLK" thru_hole circle (at -6.35 0 270) (size 2 2) (drill 1.016) (layers "*.Cu" "*.Mask") (remove_unused_layers no) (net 17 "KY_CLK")
   (solder_mask_margin 0.102))
  (pad "DT" thru_hole circle (at -3.81 0 270) (size 2 2) (drill 1.016) (layers "*.Cu" "*.Mask") (remove_unused_layers no) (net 16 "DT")
   (solder_mask_margin 0.102))
  (pad "GND" thru_hole rect (at 3.81 0 270) (size 2 2) (drill 1.016) (layers "*.Cu" "*.Mask") (remove_unused_layers no) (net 3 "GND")
   (solder_mask_margin 0.102))
  (pad "SW" thru_hole circle (at -1.27 0 270) (size 2 2) (drill 1.016) (layers "*.Cu" "*.Mask") (remove_unused_layers no) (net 15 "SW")
   (solder_mask_margin 0.102))
  (pad "VCC" thru_hole circle (at 1.27 0 270) (size 2 2) (drill 1.016) (layers "*.Cu" "*.Mask") (remove_unused_layers no) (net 31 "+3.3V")
   (solder_mask_margin 0.102)))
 (gr_rect (start 92.58 56.94) (end 157.08 145.44) (stroke (width 0.05) (type solid)) (fill no) (layer "Edge.Cuts"))
 (segment (start 144.86 116.72) (end 110.83 82.69) (width 0.5) (layer "B.Cu") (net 5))
 (segment (start 110.83 82.69) (end 104 82.69) (width 0.5) (layer "B.Cu") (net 5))
 (segment (start 98.4525 130.44) (end 98.4525 133.368128) (width 0.5) (layer "B.Cu") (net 3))
 (segment (start 108.5 68.5) (end 107.5 67.5) (width 0.5) (layer "B.Cu") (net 3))
 (segment (start 104.085372 139.001) (end 145.439 139.001) (width 0.5) (layer "B.Cu") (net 3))
 (segment (start 108.5 70) (end 108.5 68.5) (width 0.5) (layer "B.Cu") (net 3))
 (segment (start 105.97 72.53) (end 108.5 70) (width 0.5) (layer "B.Cu") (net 3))
 (segment (start 94.7343 76.0967) (end 94.7343 126.7218) (width 0.5) (layer "B.Cu") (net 3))
 (segment (start 145.439 139.001) (end 149.94 134.5) (width 0.5) (layer "B.Cu") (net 3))
 (segment (start 98.4525 133.368128) (end 104.085372 139.001) (width 0.5) (layer "B.Cu") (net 3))
 (segment (start 104 72.53) (end 105.97 72.53) (width 0.5) (layer "B.Cu") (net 3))
 (segment (start 103.331 67.5) (end 94.7343 76.0967) (width 0.5) (layer "B.Cu") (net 3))
 (segment (start 107.5 67.5) (end 103.331 67.5) (width 0.5) (layer "B.Cu") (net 3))
 (segment (start 94.7343 126.7218) (end 98.4525 130.44) (width 0.5) (layer "B.Cu") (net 3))
 (segment (start 113.37 77.61) (end 104 77.61) (width 0.5) (layer "B.Cu") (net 2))
 (segment (start 152.48 116.72) (end 113.37 77.61) (width 0.5) (layer "B.Cu") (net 2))
 (segment (start 96.7363 123.6438) (end 96.7363 119.569126) (width 0.5) (layer "B.Cu") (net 15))
 (segment (start 98.4525 125.36) (end 96.7363 123.6438) (width 0.5) (layer "B.Cu") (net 15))
 (segment (start 112.824 115.164) (end 114.38 116.72) (width 0.5) (layer "B.Cu") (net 15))
 (segment (start 96.7363 119.569126) (end 101.141426 115.164) (width 0.5) (layer "B.Cu") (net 15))
 (segment (start 101.141426 115.164) (end 112.824 115.164) (width 0.5) (layer "B.Cu") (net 15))
 (segment (start 110.83 80.15) (end 104 80.15) (width 0.5) (layer "B.Cu") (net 4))
 (segment (start 147.4 116.72) (end 110.83 80.15) (width 0.5) (layer "B.Cu") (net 4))
 (segment (start 104.34137 85.23) (end 104 85.23) (width 0.5) (layer "B.Cu") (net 8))
 (segment (start 134.7 116.72) (end 134.7 115.58863) (width 0.5) (layer "B.Cu") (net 8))
 (segment (start 134.7 115.58863) (end 104.34137 85.23) (width 0.5) (layer "B.Cu") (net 8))
 (segment (start 129.62 116.72) (end 129.62 115.58863) (width 0.5) (layer "B.Cu") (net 10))
 (segment (start 129.62 115.58863) (end 104.34137 90.31) (width 0.5) (layer "B.Cu") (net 10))
 (segment (start 104.34137 90.31) (end 104 90.31) (width 0.5) (layer "B.Cu") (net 10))
 (segment (start 98.4525 120.28) (end 103.2 120.28) (width 0.5) (layer "B.Cu") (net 17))
 (segment (start 103.2 120.28) (end 106.76 116.72) (width 0.5) (layer "B.Cu") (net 17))
 (segment (start 102.5 131.0551) (end 102.5 136) (width 0.5) (layer "B.Cu") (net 31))
 (segment (start 95.7353 93.5) (end 95.7353 77.7547) (width 0.5) (layer "B.Cu") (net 31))
 (segment (start 104 69.99) (end 103.5 69.99) (width 0.5) (layer "B.Cu") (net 31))
 (segment (start 101.4653 87.77) (end 95.7353 93.5) (width 0.5) (layer "B.Cu") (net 31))
 (segment (start 144.86 136.14) (end 143 138) (width 0.5) (layer "B.Cu") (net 31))
 (segment (start 103.5 69.99) (end 97 76.49) (width 0.5) (layer "B.Cu") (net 31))
 (segment (start 98.4525 127.9) (end 99.3449 127.9) (width 0.5) (layer "B.Cu") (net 31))
 (segment (start 143 138) (end 104.5 138) (width 0.5) (layer "B.Cu") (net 31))
 (segment (start 104.5 138) (end 102.5 136) (width 0.5) (layer "B.Cu") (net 31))
 (segment (start 95.7353 77.7547) (end 97 76.49) (width 0.5) (layer "B.Cu") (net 31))
 (segment (start 95.7353 125.1828) (end 95.7353 93.5) (width 0.5) (layer "B.Cu") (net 31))
 (segment (start 104 87.77) (end 101.4653 87.77) (width 0.5) (layer "B.Cu") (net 31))
 (segment (start 144.86 134.5) (end 144.86 136.14) (width 0.5) (layer "B.Cu") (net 31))
 (segment (start 98.4525 127.9) (end 95.7353 125.1828) (width 0.5) (layer "B.Cu") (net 31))
 (segment (start 99.3449 127.9) (end 102.5 131.0551) (width 0.5) (layer "B.Cu") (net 31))
 (segment (start 98.4525 122.82) (end 103.2 122.82) (width 0.5) (layer "B.Cu") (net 16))
 (segment (start 103.2 122.82) (end 109.3 116.72) (width 0.5) (layer "B.Cu") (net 16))
 (segment (start 155.02 116.72) (end 113.37 75.07) (width 0.5) (layer "B.Cu") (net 1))
 (segment (start 113.37 75.07) (end 104 75.07) (width 0.5) (layer "B.Cu") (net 1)))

